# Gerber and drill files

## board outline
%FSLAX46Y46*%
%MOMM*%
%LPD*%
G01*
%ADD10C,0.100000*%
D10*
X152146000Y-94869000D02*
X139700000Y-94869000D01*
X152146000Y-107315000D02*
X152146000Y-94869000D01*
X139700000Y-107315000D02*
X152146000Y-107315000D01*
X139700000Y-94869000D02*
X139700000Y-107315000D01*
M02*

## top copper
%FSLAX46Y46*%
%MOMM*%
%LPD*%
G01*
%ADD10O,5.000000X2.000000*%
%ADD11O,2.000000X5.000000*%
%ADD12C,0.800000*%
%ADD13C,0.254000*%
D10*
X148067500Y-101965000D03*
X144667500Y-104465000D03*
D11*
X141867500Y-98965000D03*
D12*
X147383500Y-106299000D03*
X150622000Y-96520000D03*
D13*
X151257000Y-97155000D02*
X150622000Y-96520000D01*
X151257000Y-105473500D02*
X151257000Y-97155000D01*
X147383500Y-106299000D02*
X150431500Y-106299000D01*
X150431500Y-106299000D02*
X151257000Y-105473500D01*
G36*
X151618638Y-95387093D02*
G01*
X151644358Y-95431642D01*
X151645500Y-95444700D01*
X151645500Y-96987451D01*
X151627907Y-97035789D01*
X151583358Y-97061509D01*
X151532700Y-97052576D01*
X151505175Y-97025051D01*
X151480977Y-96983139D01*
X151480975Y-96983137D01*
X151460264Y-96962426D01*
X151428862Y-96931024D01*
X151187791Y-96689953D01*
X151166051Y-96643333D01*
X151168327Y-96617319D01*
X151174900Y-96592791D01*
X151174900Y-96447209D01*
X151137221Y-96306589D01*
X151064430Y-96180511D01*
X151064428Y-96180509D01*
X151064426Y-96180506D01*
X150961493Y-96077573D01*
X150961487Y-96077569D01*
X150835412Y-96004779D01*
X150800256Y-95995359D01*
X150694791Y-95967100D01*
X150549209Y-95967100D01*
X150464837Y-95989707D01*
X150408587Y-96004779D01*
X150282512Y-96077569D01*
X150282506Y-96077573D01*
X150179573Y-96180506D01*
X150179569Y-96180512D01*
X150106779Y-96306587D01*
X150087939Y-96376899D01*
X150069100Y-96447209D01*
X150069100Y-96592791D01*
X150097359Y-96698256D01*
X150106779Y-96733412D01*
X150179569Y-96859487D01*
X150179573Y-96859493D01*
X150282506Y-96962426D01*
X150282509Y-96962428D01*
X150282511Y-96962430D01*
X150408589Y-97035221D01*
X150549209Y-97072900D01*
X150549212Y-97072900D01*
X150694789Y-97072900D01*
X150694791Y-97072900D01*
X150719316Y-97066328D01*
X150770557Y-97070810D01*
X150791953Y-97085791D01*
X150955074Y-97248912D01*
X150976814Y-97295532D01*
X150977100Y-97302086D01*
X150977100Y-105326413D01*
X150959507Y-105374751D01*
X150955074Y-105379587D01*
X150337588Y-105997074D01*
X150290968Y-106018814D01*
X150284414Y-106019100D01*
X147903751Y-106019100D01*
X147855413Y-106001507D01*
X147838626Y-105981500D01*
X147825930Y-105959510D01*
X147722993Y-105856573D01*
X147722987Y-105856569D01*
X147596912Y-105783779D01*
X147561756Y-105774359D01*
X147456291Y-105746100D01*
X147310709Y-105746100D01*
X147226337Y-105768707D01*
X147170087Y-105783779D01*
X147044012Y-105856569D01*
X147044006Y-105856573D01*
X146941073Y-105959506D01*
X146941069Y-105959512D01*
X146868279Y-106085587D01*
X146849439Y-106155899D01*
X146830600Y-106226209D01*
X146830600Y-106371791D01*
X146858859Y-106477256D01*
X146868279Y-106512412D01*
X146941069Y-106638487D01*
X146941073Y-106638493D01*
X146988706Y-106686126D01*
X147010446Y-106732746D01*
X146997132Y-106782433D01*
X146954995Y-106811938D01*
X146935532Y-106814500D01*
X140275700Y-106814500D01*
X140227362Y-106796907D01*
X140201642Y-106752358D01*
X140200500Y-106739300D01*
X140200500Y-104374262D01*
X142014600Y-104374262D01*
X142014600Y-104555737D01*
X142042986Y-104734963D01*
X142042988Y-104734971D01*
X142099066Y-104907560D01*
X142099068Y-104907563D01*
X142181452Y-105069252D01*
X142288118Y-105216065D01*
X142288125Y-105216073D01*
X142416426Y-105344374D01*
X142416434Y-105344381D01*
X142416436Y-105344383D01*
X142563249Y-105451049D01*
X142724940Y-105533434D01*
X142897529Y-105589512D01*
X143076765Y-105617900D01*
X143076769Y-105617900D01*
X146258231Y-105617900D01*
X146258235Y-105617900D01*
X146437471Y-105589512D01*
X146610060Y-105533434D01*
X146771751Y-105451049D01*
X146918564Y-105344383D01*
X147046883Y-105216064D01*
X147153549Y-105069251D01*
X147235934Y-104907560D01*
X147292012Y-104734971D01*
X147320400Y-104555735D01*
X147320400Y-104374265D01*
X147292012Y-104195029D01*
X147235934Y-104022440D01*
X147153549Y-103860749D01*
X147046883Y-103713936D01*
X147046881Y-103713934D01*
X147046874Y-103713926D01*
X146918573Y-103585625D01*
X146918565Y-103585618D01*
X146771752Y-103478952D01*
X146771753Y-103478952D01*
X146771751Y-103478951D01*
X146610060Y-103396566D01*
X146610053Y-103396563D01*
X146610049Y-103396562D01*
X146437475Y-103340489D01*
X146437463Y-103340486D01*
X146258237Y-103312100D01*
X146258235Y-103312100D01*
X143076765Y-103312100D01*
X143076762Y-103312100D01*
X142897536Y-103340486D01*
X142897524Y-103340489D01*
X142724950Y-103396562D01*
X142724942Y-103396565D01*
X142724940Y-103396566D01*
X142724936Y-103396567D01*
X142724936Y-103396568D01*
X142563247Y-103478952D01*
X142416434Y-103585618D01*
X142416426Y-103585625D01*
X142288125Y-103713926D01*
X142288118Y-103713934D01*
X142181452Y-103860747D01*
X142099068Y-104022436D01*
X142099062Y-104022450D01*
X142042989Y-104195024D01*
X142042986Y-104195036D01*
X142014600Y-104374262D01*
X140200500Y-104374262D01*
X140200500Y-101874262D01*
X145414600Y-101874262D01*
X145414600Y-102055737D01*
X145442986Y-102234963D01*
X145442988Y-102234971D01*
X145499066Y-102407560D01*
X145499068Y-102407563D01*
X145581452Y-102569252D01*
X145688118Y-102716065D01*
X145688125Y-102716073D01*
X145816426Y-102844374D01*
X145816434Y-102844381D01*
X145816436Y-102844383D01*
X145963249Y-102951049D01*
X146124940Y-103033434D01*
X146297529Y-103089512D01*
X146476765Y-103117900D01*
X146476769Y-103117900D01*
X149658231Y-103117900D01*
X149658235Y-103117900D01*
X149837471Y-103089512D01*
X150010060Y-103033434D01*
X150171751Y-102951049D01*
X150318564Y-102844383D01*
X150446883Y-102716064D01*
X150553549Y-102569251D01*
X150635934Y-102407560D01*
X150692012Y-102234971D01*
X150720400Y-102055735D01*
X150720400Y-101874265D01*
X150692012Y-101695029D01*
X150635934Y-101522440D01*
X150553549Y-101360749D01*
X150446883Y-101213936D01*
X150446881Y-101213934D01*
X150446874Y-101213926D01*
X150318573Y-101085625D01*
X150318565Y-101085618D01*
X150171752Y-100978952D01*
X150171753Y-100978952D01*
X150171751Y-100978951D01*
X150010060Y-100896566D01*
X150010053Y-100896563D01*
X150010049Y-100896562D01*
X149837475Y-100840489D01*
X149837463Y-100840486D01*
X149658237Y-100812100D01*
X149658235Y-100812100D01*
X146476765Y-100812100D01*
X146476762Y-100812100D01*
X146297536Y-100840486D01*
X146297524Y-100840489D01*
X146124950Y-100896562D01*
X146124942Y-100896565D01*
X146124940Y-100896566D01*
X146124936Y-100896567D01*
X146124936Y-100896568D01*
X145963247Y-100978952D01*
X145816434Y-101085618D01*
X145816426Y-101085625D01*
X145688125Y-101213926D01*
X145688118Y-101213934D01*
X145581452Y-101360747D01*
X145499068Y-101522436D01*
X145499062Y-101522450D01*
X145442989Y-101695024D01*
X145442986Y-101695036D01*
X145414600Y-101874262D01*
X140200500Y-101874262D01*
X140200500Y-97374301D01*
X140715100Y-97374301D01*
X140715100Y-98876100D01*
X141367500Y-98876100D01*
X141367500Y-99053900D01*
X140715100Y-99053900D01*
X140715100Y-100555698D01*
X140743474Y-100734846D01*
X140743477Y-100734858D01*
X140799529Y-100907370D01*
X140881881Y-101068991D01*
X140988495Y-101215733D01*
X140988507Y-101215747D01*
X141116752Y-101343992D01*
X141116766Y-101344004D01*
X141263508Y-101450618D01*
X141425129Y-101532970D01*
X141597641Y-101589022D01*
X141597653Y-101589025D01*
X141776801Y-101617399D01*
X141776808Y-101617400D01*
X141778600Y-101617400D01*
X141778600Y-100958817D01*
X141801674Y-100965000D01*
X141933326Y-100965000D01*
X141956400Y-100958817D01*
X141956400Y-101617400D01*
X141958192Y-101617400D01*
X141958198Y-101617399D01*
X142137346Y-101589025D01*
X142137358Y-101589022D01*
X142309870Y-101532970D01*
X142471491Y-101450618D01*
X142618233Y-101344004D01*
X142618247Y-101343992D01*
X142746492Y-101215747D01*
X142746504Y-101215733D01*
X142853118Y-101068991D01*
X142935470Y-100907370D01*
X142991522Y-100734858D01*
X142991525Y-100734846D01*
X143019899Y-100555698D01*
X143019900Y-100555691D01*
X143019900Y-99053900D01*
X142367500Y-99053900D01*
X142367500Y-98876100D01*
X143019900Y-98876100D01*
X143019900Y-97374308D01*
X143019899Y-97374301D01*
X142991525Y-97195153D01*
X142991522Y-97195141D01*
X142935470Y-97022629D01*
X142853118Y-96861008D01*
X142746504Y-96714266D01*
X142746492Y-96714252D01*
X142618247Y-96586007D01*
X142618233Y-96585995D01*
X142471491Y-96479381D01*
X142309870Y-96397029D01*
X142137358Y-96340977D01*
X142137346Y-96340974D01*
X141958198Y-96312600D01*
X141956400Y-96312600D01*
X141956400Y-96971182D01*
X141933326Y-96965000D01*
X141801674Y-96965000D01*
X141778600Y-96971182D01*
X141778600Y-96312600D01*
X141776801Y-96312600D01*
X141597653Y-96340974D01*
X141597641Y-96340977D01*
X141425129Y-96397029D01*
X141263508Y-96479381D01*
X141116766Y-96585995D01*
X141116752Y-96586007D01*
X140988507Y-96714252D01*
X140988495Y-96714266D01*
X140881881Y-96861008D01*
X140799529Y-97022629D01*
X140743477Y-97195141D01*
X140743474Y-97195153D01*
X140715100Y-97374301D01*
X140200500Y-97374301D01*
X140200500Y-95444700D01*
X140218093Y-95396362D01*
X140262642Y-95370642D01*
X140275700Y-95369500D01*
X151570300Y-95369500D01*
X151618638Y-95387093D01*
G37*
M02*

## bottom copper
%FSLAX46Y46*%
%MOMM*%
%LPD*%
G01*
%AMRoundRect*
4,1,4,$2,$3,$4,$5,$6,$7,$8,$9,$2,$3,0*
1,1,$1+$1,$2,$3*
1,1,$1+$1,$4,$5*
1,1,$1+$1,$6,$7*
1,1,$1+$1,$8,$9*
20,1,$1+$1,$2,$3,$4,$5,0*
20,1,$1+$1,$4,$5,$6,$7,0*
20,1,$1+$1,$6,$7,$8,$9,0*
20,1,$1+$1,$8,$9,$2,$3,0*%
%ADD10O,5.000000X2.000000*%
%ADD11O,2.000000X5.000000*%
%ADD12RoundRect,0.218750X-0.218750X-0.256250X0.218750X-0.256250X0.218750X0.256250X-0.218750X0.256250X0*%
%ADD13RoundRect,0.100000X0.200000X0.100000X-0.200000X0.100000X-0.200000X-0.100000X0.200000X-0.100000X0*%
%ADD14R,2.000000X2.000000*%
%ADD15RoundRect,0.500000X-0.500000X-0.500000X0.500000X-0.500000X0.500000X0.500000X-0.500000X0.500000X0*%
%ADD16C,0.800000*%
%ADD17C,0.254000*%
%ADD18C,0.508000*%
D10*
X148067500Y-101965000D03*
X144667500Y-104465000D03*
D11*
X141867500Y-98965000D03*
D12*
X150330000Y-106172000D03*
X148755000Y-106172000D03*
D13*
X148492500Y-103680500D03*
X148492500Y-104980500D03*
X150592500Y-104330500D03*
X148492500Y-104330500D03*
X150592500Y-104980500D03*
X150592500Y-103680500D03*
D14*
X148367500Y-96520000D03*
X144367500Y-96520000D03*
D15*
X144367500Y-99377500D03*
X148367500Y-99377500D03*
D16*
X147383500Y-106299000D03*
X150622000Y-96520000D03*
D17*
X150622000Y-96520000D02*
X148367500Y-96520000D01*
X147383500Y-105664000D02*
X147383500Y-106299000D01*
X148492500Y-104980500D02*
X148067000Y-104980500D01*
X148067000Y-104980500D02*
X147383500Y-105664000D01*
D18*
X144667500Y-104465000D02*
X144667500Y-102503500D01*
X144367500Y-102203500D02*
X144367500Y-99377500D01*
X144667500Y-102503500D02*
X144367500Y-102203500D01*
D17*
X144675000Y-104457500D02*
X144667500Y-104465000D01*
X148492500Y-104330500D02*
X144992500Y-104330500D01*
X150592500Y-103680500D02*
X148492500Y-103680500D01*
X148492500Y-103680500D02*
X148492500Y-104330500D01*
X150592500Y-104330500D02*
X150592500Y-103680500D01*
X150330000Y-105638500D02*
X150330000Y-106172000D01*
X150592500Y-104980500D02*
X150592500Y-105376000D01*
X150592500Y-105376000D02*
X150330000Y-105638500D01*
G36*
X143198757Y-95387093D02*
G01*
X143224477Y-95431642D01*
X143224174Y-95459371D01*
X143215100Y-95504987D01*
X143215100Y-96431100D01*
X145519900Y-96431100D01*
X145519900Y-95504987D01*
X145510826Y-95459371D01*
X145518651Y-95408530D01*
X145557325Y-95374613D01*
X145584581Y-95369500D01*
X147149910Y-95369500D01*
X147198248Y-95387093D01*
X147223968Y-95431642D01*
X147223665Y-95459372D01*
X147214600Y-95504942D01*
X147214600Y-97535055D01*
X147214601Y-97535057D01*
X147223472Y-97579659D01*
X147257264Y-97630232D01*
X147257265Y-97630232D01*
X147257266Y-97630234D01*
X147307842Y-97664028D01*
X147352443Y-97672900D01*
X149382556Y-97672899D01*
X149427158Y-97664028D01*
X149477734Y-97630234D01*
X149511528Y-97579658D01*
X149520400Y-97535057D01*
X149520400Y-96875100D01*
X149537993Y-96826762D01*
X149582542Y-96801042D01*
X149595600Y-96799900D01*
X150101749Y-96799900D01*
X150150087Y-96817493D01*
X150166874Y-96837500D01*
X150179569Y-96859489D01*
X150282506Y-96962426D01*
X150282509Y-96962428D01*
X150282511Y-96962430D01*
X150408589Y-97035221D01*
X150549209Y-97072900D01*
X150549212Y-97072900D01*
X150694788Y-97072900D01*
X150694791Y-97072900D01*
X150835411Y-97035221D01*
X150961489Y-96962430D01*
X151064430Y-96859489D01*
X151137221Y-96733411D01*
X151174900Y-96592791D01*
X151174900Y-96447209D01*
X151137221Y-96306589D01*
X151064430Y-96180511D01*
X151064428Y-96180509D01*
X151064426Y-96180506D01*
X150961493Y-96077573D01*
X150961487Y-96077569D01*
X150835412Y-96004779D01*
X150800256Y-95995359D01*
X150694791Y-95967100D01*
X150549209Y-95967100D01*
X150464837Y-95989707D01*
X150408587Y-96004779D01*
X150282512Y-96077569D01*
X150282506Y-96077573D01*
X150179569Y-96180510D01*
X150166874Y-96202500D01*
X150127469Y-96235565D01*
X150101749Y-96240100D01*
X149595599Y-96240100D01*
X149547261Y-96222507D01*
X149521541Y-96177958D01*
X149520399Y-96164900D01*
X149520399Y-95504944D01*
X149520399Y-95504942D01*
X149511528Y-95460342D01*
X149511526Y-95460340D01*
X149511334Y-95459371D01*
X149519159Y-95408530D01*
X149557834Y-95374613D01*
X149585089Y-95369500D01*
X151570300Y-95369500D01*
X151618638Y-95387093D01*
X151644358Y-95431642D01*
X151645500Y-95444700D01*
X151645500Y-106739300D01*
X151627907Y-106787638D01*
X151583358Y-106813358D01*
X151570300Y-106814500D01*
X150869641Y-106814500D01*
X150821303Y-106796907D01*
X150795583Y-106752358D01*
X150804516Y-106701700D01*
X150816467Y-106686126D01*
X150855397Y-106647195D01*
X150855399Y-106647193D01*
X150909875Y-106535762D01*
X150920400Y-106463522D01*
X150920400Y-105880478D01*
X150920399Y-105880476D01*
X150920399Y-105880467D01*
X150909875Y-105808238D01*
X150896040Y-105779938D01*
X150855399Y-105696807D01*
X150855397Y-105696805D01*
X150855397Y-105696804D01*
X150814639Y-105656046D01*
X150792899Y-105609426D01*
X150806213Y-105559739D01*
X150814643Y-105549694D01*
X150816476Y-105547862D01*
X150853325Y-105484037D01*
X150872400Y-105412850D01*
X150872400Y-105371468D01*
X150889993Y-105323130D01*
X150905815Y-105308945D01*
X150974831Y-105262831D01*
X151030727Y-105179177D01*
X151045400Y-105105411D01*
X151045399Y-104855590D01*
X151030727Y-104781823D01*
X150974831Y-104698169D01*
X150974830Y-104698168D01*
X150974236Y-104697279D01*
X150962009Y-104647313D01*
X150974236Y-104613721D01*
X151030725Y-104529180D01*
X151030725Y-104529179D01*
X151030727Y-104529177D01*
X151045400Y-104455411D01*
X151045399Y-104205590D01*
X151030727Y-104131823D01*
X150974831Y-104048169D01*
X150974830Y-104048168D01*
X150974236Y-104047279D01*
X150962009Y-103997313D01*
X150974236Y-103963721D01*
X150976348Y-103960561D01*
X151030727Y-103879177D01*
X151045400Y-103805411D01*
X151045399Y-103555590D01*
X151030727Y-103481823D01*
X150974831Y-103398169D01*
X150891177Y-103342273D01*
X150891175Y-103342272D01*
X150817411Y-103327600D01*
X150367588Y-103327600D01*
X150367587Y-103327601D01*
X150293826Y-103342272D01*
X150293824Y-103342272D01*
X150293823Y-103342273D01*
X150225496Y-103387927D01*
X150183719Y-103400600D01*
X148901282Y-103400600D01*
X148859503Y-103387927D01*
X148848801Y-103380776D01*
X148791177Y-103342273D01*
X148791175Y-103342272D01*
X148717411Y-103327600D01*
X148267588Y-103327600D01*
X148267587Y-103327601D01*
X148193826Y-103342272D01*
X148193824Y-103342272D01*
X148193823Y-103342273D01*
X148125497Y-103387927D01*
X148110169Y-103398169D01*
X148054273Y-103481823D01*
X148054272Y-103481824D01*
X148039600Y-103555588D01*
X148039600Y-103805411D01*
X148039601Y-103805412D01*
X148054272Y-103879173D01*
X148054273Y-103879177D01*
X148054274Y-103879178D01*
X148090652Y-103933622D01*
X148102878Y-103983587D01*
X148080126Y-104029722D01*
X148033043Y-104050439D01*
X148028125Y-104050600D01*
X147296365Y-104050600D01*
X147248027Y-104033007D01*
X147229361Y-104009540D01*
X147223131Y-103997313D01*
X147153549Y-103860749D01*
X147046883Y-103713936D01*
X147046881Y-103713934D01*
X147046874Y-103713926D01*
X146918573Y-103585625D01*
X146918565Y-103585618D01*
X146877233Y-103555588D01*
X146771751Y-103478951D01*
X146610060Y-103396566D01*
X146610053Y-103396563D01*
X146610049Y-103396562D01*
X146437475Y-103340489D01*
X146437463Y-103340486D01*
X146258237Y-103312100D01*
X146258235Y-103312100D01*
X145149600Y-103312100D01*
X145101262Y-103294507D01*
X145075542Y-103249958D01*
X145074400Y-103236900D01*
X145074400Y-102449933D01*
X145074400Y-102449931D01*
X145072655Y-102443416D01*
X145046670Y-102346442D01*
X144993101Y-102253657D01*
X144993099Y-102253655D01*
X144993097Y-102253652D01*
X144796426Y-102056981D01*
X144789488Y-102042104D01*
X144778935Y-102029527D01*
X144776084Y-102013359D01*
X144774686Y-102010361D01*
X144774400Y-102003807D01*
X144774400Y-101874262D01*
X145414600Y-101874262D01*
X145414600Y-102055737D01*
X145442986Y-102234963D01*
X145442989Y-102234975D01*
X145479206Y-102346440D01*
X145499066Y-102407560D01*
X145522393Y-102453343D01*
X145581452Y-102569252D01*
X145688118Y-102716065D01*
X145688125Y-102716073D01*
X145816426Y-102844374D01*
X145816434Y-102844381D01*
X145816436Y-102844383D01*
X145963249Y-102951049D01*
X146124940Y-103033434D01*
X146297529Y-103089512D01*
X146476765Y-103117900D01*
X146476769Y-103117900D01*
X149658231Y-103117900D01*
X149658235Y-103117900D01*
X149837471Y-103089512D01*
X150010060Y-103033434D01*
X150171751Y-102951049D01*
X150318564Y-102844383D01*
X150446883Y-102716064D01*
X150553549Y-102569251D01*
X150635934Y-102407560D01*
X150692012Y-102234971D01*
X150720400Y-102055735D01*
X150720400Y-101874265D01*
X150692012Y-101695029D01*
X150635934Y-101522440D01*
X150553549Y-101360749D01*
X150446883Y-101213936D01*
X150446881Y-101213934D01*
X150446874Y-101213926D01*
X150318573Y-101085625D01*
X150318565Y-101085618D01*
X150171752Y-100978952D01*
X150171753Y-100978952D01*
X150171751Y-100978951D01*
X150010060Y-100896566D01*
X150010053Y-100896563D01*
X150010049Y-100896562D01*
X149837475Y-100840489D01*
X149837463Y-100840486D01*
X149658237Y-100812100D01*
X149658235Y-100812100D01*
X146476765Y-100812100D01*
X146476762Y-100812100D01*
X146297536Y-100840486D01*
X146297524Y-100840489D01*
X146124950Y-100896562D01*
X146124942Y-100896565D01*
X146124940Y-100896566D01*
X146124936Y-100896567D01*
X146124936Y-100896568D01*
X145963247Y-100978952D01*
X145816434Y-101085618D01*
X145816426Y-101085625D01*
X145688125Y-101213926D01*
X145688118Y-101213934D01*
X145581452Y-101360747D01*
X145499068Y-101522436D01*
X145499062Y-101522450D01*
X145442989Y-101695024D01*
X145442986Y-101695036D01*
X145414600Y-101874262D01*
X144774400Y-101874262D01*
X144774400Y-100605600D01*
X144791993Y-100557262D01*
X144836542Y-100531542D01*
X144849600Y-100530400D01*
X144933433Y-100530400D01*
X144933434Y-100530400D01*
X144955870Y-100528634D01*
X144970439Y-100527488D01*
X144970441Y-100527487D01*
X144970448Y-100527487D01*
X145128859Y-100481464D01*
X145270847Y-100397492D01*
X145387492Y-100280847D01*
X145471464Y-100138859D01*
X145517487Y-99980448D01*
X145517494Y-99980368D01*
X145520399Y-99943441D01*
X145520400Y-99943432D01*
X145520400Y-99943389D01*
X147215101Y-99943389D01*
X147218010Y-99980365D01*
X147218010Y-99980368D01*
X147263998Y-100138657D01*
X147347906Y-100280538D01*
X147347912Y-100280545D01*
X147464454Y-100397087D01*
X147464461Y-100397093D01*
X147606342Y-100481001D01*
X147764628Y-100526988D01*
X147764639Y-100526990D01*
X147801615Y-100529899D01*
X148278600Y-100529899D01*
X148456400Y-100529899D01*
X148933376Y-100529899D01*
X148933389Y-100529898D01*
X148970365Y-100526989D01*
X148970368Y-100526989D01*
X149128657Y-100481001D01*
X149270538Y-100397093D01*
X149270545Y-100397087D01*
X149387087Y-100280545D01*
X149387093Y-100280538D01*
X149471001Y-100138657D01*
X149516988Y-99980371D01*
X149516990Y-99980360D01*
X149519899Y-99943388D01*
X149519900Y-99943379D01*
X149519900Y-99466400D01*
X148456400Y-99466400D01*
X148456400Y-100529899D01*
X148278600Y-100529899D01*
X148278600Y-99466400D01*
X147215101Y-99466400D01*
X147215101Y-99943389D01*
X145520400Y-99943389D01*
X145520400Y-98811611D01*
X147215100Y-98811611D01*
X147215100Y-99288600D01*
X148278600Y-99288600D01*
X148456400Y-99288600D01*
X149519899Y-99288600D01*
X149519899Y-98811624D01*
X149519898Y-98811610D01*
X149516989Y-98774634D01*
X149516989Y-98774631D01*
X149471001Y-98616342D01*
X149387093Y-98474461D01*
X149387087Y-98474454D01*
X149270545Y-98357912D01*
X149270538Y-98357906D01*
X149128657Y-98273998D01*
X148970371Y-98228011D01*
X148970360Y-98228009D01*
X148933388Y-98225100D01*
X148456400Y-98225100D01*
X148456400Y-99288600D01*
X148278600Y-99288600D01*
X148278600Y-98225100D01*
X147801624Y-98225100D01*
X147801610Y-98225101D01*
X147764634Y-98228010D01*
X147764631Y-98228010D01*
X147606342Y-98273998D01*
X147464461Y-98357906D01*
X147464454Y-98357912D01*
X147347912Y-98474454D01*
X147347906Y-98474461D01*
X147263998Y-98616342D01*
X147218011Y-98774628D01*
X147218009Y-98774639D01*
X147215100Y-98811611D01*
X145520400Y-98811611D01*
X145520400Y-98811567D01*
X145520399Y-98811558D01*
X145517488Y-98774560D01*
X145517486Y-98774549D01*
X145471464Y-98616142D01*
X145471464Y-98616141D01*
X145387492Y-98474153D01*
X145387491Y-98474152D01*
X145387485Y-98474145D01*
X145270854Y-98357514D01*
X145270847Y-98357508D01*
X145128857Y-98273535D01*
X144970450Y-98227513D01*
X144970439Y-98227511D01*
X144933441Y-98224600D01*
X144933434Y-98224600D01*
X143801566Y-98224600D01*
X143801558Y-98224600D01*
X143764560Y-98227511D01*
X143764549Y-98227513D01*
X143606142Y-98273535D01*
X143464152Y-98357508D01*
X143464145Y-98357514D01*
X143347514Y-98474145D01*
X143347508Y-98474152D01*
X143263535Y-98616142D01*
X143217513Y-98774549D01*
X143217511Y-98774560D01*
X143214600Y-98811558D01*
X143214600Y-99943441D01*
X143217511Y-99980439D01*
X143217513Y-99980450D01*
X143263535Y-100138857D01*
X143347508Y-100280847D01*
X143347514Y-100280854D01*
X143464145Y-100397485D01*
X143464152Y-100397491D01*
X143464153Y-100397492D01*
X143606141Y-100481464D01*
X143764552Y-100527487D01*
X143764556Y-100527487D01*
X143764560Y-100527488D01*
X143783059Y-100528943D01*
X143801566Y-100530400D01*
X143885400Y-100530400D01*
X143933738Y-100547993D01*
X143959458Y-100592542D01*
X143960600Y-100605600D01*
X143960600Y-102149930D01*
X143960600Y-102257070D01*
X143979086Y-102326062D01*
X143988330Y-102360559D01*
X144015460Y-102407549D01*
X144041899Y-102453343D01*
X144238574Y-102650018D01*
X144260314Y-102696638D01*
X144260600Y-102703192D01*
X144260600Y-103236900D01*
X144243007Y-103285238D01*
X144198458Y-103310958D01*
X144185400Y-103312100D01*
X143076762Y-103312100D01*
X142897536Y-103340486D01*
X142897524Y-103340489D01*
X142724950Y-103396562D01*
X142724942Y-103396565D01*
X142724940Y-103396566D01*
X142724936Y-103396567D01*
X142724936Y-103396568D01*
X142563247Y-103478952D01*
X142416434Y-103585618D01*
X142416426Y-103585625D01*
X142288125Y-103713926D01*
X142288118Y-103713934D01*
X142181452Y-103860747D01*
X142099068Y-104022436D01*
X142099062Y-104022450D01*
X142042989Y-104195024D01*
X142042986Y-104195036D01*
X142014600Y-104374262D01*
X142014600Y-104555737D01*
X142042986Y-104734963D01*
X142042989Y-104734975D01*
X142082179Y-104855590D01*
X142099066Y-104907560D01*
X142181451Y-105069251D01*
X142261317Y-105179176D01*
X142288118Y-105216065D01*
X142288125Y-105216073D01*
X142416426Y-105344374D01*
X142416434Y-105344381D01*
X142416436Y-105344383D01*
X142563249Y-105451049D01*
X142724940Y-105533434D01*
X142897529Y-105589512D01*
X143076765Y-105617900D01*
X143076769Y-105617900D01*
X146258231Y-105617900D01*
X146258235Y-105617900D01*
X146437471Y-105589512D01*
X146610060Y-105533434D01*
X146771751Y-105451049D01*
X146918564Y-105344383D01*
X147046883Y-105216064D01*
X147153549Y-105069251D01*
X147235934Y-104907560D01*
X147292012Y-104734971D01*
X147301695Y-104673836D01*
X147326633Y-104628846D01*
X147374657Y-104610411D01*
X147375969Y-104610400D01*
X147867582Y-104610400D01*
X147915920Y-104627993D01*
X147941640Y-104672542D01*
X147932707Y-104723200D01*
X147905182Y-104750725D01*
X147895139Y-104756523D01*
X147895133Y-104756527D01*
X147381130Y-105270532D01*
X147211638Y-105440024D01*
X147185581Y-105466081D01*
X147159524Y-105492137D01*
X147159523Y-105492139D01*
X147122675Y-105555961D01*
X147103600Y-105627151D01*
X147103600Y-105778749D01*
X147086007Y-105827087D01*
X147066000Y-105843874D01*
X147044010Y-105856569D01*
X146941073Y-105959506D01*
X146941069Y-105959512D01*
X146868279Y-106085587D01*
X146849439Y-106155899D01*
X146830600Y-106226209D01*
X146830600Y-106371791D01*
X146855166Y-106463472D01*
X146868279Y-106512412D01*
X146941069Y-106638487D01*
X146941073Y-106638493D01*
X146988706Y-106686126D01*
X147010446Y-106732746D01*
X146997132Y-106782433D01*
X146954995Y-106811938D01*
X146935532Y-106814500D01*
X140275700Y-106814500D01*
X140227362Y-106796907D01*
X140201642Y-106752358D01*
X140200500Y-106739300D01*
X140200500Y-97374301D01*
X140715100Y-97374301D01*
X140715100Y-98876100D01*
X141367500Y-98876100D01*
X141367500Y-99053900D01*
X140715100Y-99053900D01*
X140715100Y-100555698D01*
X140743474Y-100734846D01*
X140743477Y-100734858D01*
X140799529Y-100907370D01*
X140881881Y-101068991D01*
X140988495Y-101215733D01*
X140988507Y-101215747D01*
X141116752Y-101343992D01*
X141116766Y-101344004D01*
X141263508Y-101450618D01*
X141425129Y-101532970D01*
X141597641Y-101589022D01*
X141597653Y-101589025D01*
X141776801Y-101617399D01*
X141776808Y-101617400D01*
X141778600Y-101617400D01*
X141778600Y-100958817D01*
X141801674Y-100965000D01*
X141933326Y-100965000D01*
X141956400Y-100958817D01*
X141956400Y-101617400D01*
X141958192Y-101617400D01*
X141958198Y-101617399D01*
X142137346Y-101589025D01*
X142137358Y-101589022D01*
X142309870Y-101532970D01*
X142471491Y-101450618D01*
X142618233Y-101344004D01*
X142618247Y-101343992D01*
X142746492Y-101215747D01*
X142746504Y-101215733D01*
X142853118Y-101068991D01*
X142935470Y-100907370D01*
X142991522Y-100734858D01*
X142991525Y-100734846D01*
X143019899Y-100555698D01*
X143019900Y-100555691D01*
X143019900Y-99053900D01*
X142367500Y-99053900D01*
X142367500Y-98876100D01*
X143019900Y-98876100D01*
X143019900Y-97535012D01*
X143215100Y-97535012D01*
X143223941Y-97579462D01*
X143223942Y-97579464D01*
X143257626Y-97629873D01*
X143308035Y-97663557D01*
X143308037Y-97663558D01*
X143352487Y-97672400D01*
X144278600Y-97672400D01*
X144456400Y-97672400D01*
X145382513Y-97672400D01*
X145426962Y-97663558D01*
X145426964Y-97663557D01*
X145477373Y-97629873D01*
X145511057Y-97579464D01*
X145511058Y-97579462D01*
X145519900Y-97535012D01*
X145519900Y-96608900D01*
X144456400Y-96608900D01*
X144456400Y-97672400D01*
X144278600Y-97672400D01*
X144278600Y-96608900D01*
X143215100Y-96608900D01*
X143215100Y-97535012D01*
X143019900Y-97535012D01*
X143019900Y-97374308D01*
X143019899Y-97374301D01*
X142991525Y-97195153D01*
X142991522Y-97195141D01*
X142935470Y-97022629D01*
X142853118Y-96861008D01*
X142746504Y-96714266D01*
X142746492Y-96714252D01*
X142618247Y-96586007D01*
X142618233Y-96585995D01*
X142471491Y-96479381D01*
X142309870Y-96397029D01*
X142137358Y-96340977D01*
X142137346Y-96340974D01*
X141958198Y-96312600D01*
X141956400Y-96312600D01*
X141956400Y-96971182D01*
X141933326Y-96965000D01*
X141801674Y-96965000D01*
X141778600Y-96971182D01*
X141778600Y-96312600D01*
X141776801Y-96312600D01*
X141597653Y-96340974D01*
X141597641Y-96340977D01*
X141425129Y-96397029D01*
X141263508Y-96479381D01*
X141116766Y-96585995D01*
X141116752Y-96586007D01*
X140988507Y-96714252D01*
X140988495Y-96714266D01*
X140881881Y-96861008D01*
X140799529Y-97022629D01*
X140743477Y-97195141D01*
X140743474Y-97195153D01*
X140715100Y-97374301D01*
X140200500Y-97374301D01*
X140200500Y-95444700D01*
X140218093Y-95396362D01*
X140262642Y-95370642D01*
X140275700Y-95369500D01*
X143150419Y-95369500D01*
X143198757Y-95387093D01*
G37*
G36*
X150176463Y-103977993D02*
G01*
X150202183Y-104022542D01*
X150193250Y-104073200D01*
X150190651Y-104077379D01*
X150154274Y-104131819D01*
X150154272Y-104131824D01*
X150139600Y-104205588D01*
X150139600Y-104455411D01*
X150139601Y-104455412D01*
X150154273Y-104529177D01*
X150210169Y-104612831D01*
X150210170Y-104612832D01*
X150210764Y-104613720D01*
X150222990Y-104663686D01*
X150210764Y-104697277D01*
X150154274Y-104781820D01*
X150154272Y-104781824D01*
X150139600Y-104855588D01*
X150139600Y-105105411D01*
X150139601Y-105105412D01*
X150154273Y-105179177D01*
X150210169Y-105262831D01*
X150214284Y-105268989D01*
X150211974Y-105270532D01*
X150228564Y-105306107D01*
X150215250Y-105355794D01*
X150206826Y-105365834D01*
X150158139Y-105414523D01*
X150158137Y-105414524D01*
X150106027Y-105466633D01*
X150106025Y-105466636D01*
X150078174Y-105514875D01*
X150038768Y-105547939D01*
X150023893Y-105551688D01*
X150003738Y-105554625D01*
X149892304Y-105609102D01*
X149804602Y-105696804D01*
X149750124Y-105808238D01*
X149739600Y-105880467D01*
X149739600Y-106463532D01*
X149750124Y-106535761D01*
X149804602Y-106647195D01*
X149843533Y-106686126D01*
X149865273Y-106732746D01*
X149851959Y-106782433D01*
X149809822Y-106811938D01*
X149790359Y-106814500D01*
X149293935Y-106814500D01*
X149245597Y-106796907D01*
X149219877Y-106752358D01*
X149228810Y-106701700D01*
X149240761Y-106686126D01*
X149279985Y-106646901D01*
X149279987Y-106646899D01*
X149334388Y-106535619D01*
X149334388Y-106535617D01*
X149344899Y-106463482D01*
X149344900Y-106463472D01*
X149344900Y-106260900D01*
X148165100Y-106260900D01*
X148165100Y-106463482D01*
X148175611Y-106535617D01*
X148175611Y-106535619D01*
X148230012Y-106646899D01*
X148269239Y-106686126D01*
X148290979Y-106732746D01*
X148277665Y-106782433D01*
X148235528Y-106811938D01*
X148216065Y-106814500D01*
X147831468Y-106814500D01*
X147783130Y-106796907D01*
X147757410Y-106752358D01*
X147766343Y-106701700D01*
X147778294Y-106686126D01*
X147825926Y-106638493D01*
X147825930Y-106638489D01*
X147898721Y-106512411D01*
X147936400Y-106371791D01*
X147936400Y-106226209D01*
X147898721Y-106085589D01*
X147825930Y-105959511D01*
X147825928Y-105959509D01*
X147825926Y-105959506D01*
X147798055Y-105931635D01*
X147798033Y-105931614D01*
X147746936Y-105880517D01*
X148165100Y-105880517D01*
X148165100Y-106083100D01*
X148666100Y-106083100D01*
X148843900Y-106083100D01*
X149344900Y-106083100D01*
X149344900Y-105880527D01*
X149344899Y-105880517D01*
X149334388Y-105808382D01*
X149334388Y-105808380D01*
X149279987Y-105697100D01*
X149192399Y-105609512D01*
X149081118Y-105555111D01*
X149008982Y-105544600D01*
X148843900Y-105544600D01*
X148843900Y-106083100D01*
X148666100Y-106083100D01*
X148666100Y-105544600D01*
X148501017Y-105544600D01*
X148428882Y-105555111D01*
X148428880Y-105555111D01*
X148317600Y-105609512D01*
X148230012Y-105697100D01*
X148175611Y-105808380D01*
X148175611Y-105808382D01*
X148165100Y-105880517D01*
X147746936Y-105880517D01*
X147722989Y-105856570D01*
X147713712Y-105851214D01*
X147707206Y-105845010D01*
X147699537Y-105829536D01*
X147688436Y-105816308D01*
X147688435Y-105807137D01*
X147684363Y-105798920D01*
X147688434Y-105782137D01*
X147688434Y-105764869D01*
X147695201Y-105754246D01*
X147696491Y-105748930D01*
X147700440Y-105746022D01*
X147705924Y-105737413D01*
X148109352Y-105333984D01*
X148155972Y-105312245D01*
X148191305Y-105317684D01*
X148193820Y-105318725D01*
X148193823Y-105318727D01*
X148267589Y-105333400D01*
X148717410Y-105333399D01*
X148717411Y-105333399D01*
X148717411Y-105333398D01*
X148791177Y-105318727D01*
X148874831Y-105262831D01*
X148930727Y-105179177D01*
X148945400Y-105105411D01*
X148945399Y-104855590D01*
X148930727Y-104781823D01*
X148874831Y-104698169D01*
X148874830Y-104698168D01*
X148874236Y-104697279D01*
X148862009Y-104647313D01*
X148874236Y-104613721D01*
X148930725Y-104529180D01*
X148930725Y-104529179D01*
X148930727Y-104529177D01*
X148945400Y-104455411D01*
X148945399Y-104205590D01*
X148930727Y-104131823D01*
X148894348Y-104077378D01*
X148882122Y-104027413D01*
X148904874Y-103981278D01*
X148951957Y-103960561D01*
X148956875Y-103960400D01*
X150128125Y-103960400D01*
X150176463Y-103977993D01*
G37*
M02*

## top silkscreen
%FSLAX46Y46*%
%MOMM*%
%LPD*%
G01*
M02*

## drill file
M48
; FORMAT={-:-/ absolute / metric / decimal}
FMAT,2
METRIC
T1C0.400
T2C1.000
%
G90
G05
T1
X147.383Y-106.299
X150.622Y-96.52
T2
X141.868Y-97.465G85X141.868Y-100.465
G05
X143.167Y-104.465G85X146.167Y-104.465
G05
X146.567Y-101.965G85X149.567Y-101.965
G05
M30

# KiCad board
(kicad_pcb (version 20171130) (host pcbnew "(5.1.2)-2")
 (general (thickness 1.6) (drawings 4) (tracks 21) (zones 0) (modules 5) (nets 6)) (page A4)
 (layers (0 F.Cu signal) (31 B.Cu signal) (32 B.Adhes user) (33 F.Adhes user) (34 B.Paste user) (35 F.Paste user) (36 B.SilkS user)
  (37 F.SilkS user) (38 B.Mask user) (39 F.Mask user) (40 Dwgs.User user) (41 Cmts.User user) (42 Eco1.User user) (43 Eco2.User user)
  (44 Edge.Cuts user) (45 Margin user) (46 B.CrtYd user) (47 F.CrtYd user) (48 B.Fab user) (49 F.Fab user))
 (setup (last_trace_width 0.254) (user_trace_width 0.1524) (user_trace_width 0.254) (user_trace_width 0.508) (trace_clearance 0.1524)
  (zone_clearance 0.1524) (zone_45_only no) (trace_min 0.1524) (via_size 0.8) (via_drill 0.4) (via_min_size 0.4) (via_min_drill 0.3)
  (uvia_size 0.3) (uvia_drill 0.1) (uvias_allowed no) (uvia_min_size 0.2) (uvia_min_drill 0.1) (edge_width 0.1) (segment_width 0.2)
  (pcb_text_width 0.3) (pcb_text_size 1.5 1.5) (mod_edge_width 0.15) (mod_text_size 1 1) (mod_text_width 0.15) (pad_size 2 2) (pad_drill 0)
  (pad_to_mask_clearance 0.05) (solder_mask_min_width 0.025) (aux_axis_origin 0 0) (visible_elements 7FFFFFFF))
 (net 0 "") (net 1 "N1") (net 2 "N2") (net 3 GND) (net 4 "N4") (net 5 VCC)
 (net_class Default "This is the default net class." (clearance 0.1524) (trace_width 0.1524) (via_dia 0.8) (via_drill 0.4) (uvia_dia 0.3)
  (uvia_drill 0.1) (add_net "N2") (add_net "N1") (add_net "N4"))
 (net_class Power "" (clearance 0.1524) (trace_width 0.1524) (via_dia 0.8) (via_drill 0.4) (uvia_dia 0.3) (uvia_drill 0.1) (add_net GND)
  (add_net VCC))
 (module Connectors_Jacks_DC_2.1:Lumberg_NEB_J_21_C (layer F.Cu) (at 146.3675 100.965)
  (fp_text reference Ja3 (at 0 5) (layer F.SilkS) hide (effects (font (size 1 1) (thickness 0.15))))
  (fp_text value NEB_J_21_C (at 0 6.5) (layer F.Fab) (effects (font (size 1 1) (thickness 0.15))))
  (pad 3 thru_hole oval (at 1.7 1) (size 5 2) (drill oval 4 1) (layers *.Cu *.Mask) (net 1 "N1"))
  (pad 2 thru_hole oval (at -1.7 3.5) (size 5 2) (drill oval 4 1) (layers *.Cu *.Mask) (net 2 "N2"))
  (pad 1 thru_hole oval (at -4.5 -2) (size 2 5) (drill oval 1 4) (layers *.Cu *.Mask) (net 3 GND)))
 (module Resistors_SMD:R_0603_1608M (layer B.Cu) (at 149.5425 106.172)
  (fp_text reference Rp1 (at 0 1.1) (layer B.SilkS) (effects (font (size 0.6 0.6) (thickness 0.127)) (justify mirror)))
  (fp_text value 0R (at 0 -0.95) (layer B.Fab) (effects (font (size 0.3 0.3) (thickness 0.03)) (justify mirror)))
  (pad 2 smd roundrect (at 0.7875 0) (size 0.875 0.95) (layers B.Cu B.Paste B.Mask) (roundrect_rratio 0.25) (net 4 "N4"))
  (pad 1 smd roundrect (at -0.7875 0) (size 0.875 0.95) (layers B.Cu B.Paste B.Mask) (roundrect_rratio 0.25) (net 3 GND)))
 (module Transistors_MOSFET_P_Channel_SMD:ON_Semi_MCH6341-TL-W (layer B.Cu) (at 149.5425 104.3305 180)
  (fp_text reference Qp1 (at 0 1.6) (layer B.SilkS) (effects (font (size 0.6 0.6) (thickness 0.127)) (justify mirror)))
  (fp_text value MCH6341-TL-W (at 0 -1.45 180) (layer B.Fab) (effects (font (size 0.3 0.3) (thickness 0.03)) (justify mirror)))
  (pad 6 smd roundrect (at 1.05 0.65 180) (size 0.6 0.4) (layers B.Cu B.Paste B.Mask) (roundrect_rratio 0.25) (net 2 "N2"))
  (pad 4 smd roundrect (at 1.05 -0.65 180) (size 0.6 0.4) (layers B.Cu B.Paste B.Mask) (roundrect_rratio 0.25) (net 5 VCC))
  (pad 2 smd roundrect (at -1.05 0 180) (size 0.6 0.4) (layers B.Cu B.Paste B.Mask) (roundrect_rratio 0.25) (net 2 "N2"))
  (pad 5 smd roundrect (at 1.05 0 180) (size 0.6 0.4) (layers B.Cu B.Paste B.Mask) (roundrect_rratio 0.25) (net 2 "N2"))
  (pad 3 smd roundrect (at -1.05 -0.65 180) (size 0.6 0.4) (layers B.Cu B.Paste B.Mask) (roundrect_rratio 0.25) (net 4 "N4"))
  (pad 1 smd roundrect (at -1.05 0.65 180) (size 0.6 0.4) (layers B.Cu B.Paste B.Mask) (roundrect_rratio 0.25) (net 2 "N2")))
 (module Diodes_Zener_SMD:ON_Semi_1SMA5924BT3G (layer B.Cu) (at 146.3675 96.52 180)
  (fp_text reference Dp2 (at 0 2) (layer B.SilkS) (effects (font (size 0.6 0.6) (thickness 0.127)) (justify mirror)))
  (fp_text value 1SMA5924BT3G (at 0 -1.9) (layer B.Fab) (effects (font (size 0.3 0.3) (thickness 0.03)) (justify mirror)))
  (pad 2 smd rect (at -2 0 180) (size 2 2) (layers B.Cu B.Paste B.Mask) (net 5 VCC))
  (pad 1 smd rect (at 2 0 180) (size 2 2) (layers B.Cu B.Paste B.Mask) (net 3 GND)))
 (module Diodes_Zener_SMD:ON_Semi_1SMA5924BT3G (layer B.Cu) (at 146.3675 99.3775)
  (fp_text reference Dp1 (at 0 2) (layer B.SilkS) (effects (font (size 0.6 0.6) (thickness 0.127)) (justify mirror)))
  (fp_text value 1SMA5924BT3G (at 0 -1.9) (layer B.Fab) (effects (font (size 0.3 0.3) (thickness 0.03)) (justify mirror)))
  (pad 2 smd roundrect (at -2 0) (size 2 2) (layers B.Cu B.Paste B.Mask) (roundrect_rratio 0.25) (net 2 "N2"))
  (pad 1 smd roundrect (at 2 0) (size 2 2) (layers B.Cu B.Paste B.Mask) (roundrect_rratio 0.25) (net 3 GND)))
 (gr_line (start 152.146 94.869) (end 139.7 94.869) (layer Edge.Cuts) (width 0.1))
 (gr_line (start 152.146 107.315) (end 152.146 94.869) (layer Edge.Cuts) (width 0.1))
 (gr_line (start 139.7 107.315) (end 152.146 107.315) (layer Edge.Cuts) (width 0.1))
 (gr_line (start 139.7 94.869) (end 139.7 107.315) (layer Edge.Cuts) (width 0.1))
 (via (at 147.3835 106.299) (size 0.8) (drill 0.4) (layers F.Cu B.Cu) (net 5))
 (via (at 150.622 96.52) (size 0.8) (drill 0.4) (layers F.Cu B.Cu) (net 5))
 (segment (start 150.622 96.52) (end 148.3675 96.52) (width 0.254) (layer B.Cu) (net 5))
 (segment (start 147.3835 105.664) (end 147.3835 106.299) (width 0.254) (layer B.Cu) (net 5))
 (segment (start 148.4925 104.9805) (end 148.067 104.9805) (width 0.254) (layer B.Cu) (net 5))
 (segment (start 148.067 104.9805) (end 147.3835 105.664) (width 0.254) (layer B.Cu) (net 5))
 (segment (start 151.257 97.155) (end 150.622 96.52) (width 0.254) (layer F.Cu) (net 5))
 (segment (start 151.257 105.4735) (end 151.257 97.155) (width 0.254) (layer F.Cu) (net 5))
 (segment (start 147.3835 106.299) (end 150.4315 106.299) (width 0.254) (layer F.Cu) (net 5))
 (segment (start 150.4315 106.299) (end 151.257 105.4735) (width 0.254) (layer F.Cu) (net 5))
 (segment (start 144.6675 104.465) (end 144.6675 102.5035) (width 0.508) (layer B.Cu) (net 2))
 (segment (start 144.3675 102.2035) (end 144.3675 99.3775) (width 0.508) (layer B.Cu) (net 2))
 (segment (start 144.6675 102.5035) (end 144.3675 102.2035) (width 0.508) (layer B.Cu) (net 2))
 (segment (start 144.675 104.4575) (end 144.6675 104.465) (width 0.254) (layer B.Cu) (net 2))
 (segment (start 148.4925 104.3305) (end 144.9925 104.3305) (width 0.254) (layer B.Cu) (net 2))
 (segment (start 150.5925 103.6805) (end 148.4925 103.6805) (width 0.254) (layer B.Cu) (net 2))
 (segment (start 148.4925 103.6805) (end 148.4925 104.3305) (width 0.254) (layer B.Cu) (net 2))
 (segment (start 150.5925 104.3305) (end 150.5925 103.6805) (width 0.254) (layer B.Cu) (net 2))
 (segment (start 150.33 105.6385) (end 150.33 106.172) (width 0.254) (layer B.Cu) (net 4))
 (segment (start 150.5925 104.9805) (end 150.5925 105.376) (width 0.254) (layer B.Cu) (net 4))
 (segment (start 150.5925 105.376) (end 150.33 105.6385) (width 0.254) (layer B.Cu) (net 4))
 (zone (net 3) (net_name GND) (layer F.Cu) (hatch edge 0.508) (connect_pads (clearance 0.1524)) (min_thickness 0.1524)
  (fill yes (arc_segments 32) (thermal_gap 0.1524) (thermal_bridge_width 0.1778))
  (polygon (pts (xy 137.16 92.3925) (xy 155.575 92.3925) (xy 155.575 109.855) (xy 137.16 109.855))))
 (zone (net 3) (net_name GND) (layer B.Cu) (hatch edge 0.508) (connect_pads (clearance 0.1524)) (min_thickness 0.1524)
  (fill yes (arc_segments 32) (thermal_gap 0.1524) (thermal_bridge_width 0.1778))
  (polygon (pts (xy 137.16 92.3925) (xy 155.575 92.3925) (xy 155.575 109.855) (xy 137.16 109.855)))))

